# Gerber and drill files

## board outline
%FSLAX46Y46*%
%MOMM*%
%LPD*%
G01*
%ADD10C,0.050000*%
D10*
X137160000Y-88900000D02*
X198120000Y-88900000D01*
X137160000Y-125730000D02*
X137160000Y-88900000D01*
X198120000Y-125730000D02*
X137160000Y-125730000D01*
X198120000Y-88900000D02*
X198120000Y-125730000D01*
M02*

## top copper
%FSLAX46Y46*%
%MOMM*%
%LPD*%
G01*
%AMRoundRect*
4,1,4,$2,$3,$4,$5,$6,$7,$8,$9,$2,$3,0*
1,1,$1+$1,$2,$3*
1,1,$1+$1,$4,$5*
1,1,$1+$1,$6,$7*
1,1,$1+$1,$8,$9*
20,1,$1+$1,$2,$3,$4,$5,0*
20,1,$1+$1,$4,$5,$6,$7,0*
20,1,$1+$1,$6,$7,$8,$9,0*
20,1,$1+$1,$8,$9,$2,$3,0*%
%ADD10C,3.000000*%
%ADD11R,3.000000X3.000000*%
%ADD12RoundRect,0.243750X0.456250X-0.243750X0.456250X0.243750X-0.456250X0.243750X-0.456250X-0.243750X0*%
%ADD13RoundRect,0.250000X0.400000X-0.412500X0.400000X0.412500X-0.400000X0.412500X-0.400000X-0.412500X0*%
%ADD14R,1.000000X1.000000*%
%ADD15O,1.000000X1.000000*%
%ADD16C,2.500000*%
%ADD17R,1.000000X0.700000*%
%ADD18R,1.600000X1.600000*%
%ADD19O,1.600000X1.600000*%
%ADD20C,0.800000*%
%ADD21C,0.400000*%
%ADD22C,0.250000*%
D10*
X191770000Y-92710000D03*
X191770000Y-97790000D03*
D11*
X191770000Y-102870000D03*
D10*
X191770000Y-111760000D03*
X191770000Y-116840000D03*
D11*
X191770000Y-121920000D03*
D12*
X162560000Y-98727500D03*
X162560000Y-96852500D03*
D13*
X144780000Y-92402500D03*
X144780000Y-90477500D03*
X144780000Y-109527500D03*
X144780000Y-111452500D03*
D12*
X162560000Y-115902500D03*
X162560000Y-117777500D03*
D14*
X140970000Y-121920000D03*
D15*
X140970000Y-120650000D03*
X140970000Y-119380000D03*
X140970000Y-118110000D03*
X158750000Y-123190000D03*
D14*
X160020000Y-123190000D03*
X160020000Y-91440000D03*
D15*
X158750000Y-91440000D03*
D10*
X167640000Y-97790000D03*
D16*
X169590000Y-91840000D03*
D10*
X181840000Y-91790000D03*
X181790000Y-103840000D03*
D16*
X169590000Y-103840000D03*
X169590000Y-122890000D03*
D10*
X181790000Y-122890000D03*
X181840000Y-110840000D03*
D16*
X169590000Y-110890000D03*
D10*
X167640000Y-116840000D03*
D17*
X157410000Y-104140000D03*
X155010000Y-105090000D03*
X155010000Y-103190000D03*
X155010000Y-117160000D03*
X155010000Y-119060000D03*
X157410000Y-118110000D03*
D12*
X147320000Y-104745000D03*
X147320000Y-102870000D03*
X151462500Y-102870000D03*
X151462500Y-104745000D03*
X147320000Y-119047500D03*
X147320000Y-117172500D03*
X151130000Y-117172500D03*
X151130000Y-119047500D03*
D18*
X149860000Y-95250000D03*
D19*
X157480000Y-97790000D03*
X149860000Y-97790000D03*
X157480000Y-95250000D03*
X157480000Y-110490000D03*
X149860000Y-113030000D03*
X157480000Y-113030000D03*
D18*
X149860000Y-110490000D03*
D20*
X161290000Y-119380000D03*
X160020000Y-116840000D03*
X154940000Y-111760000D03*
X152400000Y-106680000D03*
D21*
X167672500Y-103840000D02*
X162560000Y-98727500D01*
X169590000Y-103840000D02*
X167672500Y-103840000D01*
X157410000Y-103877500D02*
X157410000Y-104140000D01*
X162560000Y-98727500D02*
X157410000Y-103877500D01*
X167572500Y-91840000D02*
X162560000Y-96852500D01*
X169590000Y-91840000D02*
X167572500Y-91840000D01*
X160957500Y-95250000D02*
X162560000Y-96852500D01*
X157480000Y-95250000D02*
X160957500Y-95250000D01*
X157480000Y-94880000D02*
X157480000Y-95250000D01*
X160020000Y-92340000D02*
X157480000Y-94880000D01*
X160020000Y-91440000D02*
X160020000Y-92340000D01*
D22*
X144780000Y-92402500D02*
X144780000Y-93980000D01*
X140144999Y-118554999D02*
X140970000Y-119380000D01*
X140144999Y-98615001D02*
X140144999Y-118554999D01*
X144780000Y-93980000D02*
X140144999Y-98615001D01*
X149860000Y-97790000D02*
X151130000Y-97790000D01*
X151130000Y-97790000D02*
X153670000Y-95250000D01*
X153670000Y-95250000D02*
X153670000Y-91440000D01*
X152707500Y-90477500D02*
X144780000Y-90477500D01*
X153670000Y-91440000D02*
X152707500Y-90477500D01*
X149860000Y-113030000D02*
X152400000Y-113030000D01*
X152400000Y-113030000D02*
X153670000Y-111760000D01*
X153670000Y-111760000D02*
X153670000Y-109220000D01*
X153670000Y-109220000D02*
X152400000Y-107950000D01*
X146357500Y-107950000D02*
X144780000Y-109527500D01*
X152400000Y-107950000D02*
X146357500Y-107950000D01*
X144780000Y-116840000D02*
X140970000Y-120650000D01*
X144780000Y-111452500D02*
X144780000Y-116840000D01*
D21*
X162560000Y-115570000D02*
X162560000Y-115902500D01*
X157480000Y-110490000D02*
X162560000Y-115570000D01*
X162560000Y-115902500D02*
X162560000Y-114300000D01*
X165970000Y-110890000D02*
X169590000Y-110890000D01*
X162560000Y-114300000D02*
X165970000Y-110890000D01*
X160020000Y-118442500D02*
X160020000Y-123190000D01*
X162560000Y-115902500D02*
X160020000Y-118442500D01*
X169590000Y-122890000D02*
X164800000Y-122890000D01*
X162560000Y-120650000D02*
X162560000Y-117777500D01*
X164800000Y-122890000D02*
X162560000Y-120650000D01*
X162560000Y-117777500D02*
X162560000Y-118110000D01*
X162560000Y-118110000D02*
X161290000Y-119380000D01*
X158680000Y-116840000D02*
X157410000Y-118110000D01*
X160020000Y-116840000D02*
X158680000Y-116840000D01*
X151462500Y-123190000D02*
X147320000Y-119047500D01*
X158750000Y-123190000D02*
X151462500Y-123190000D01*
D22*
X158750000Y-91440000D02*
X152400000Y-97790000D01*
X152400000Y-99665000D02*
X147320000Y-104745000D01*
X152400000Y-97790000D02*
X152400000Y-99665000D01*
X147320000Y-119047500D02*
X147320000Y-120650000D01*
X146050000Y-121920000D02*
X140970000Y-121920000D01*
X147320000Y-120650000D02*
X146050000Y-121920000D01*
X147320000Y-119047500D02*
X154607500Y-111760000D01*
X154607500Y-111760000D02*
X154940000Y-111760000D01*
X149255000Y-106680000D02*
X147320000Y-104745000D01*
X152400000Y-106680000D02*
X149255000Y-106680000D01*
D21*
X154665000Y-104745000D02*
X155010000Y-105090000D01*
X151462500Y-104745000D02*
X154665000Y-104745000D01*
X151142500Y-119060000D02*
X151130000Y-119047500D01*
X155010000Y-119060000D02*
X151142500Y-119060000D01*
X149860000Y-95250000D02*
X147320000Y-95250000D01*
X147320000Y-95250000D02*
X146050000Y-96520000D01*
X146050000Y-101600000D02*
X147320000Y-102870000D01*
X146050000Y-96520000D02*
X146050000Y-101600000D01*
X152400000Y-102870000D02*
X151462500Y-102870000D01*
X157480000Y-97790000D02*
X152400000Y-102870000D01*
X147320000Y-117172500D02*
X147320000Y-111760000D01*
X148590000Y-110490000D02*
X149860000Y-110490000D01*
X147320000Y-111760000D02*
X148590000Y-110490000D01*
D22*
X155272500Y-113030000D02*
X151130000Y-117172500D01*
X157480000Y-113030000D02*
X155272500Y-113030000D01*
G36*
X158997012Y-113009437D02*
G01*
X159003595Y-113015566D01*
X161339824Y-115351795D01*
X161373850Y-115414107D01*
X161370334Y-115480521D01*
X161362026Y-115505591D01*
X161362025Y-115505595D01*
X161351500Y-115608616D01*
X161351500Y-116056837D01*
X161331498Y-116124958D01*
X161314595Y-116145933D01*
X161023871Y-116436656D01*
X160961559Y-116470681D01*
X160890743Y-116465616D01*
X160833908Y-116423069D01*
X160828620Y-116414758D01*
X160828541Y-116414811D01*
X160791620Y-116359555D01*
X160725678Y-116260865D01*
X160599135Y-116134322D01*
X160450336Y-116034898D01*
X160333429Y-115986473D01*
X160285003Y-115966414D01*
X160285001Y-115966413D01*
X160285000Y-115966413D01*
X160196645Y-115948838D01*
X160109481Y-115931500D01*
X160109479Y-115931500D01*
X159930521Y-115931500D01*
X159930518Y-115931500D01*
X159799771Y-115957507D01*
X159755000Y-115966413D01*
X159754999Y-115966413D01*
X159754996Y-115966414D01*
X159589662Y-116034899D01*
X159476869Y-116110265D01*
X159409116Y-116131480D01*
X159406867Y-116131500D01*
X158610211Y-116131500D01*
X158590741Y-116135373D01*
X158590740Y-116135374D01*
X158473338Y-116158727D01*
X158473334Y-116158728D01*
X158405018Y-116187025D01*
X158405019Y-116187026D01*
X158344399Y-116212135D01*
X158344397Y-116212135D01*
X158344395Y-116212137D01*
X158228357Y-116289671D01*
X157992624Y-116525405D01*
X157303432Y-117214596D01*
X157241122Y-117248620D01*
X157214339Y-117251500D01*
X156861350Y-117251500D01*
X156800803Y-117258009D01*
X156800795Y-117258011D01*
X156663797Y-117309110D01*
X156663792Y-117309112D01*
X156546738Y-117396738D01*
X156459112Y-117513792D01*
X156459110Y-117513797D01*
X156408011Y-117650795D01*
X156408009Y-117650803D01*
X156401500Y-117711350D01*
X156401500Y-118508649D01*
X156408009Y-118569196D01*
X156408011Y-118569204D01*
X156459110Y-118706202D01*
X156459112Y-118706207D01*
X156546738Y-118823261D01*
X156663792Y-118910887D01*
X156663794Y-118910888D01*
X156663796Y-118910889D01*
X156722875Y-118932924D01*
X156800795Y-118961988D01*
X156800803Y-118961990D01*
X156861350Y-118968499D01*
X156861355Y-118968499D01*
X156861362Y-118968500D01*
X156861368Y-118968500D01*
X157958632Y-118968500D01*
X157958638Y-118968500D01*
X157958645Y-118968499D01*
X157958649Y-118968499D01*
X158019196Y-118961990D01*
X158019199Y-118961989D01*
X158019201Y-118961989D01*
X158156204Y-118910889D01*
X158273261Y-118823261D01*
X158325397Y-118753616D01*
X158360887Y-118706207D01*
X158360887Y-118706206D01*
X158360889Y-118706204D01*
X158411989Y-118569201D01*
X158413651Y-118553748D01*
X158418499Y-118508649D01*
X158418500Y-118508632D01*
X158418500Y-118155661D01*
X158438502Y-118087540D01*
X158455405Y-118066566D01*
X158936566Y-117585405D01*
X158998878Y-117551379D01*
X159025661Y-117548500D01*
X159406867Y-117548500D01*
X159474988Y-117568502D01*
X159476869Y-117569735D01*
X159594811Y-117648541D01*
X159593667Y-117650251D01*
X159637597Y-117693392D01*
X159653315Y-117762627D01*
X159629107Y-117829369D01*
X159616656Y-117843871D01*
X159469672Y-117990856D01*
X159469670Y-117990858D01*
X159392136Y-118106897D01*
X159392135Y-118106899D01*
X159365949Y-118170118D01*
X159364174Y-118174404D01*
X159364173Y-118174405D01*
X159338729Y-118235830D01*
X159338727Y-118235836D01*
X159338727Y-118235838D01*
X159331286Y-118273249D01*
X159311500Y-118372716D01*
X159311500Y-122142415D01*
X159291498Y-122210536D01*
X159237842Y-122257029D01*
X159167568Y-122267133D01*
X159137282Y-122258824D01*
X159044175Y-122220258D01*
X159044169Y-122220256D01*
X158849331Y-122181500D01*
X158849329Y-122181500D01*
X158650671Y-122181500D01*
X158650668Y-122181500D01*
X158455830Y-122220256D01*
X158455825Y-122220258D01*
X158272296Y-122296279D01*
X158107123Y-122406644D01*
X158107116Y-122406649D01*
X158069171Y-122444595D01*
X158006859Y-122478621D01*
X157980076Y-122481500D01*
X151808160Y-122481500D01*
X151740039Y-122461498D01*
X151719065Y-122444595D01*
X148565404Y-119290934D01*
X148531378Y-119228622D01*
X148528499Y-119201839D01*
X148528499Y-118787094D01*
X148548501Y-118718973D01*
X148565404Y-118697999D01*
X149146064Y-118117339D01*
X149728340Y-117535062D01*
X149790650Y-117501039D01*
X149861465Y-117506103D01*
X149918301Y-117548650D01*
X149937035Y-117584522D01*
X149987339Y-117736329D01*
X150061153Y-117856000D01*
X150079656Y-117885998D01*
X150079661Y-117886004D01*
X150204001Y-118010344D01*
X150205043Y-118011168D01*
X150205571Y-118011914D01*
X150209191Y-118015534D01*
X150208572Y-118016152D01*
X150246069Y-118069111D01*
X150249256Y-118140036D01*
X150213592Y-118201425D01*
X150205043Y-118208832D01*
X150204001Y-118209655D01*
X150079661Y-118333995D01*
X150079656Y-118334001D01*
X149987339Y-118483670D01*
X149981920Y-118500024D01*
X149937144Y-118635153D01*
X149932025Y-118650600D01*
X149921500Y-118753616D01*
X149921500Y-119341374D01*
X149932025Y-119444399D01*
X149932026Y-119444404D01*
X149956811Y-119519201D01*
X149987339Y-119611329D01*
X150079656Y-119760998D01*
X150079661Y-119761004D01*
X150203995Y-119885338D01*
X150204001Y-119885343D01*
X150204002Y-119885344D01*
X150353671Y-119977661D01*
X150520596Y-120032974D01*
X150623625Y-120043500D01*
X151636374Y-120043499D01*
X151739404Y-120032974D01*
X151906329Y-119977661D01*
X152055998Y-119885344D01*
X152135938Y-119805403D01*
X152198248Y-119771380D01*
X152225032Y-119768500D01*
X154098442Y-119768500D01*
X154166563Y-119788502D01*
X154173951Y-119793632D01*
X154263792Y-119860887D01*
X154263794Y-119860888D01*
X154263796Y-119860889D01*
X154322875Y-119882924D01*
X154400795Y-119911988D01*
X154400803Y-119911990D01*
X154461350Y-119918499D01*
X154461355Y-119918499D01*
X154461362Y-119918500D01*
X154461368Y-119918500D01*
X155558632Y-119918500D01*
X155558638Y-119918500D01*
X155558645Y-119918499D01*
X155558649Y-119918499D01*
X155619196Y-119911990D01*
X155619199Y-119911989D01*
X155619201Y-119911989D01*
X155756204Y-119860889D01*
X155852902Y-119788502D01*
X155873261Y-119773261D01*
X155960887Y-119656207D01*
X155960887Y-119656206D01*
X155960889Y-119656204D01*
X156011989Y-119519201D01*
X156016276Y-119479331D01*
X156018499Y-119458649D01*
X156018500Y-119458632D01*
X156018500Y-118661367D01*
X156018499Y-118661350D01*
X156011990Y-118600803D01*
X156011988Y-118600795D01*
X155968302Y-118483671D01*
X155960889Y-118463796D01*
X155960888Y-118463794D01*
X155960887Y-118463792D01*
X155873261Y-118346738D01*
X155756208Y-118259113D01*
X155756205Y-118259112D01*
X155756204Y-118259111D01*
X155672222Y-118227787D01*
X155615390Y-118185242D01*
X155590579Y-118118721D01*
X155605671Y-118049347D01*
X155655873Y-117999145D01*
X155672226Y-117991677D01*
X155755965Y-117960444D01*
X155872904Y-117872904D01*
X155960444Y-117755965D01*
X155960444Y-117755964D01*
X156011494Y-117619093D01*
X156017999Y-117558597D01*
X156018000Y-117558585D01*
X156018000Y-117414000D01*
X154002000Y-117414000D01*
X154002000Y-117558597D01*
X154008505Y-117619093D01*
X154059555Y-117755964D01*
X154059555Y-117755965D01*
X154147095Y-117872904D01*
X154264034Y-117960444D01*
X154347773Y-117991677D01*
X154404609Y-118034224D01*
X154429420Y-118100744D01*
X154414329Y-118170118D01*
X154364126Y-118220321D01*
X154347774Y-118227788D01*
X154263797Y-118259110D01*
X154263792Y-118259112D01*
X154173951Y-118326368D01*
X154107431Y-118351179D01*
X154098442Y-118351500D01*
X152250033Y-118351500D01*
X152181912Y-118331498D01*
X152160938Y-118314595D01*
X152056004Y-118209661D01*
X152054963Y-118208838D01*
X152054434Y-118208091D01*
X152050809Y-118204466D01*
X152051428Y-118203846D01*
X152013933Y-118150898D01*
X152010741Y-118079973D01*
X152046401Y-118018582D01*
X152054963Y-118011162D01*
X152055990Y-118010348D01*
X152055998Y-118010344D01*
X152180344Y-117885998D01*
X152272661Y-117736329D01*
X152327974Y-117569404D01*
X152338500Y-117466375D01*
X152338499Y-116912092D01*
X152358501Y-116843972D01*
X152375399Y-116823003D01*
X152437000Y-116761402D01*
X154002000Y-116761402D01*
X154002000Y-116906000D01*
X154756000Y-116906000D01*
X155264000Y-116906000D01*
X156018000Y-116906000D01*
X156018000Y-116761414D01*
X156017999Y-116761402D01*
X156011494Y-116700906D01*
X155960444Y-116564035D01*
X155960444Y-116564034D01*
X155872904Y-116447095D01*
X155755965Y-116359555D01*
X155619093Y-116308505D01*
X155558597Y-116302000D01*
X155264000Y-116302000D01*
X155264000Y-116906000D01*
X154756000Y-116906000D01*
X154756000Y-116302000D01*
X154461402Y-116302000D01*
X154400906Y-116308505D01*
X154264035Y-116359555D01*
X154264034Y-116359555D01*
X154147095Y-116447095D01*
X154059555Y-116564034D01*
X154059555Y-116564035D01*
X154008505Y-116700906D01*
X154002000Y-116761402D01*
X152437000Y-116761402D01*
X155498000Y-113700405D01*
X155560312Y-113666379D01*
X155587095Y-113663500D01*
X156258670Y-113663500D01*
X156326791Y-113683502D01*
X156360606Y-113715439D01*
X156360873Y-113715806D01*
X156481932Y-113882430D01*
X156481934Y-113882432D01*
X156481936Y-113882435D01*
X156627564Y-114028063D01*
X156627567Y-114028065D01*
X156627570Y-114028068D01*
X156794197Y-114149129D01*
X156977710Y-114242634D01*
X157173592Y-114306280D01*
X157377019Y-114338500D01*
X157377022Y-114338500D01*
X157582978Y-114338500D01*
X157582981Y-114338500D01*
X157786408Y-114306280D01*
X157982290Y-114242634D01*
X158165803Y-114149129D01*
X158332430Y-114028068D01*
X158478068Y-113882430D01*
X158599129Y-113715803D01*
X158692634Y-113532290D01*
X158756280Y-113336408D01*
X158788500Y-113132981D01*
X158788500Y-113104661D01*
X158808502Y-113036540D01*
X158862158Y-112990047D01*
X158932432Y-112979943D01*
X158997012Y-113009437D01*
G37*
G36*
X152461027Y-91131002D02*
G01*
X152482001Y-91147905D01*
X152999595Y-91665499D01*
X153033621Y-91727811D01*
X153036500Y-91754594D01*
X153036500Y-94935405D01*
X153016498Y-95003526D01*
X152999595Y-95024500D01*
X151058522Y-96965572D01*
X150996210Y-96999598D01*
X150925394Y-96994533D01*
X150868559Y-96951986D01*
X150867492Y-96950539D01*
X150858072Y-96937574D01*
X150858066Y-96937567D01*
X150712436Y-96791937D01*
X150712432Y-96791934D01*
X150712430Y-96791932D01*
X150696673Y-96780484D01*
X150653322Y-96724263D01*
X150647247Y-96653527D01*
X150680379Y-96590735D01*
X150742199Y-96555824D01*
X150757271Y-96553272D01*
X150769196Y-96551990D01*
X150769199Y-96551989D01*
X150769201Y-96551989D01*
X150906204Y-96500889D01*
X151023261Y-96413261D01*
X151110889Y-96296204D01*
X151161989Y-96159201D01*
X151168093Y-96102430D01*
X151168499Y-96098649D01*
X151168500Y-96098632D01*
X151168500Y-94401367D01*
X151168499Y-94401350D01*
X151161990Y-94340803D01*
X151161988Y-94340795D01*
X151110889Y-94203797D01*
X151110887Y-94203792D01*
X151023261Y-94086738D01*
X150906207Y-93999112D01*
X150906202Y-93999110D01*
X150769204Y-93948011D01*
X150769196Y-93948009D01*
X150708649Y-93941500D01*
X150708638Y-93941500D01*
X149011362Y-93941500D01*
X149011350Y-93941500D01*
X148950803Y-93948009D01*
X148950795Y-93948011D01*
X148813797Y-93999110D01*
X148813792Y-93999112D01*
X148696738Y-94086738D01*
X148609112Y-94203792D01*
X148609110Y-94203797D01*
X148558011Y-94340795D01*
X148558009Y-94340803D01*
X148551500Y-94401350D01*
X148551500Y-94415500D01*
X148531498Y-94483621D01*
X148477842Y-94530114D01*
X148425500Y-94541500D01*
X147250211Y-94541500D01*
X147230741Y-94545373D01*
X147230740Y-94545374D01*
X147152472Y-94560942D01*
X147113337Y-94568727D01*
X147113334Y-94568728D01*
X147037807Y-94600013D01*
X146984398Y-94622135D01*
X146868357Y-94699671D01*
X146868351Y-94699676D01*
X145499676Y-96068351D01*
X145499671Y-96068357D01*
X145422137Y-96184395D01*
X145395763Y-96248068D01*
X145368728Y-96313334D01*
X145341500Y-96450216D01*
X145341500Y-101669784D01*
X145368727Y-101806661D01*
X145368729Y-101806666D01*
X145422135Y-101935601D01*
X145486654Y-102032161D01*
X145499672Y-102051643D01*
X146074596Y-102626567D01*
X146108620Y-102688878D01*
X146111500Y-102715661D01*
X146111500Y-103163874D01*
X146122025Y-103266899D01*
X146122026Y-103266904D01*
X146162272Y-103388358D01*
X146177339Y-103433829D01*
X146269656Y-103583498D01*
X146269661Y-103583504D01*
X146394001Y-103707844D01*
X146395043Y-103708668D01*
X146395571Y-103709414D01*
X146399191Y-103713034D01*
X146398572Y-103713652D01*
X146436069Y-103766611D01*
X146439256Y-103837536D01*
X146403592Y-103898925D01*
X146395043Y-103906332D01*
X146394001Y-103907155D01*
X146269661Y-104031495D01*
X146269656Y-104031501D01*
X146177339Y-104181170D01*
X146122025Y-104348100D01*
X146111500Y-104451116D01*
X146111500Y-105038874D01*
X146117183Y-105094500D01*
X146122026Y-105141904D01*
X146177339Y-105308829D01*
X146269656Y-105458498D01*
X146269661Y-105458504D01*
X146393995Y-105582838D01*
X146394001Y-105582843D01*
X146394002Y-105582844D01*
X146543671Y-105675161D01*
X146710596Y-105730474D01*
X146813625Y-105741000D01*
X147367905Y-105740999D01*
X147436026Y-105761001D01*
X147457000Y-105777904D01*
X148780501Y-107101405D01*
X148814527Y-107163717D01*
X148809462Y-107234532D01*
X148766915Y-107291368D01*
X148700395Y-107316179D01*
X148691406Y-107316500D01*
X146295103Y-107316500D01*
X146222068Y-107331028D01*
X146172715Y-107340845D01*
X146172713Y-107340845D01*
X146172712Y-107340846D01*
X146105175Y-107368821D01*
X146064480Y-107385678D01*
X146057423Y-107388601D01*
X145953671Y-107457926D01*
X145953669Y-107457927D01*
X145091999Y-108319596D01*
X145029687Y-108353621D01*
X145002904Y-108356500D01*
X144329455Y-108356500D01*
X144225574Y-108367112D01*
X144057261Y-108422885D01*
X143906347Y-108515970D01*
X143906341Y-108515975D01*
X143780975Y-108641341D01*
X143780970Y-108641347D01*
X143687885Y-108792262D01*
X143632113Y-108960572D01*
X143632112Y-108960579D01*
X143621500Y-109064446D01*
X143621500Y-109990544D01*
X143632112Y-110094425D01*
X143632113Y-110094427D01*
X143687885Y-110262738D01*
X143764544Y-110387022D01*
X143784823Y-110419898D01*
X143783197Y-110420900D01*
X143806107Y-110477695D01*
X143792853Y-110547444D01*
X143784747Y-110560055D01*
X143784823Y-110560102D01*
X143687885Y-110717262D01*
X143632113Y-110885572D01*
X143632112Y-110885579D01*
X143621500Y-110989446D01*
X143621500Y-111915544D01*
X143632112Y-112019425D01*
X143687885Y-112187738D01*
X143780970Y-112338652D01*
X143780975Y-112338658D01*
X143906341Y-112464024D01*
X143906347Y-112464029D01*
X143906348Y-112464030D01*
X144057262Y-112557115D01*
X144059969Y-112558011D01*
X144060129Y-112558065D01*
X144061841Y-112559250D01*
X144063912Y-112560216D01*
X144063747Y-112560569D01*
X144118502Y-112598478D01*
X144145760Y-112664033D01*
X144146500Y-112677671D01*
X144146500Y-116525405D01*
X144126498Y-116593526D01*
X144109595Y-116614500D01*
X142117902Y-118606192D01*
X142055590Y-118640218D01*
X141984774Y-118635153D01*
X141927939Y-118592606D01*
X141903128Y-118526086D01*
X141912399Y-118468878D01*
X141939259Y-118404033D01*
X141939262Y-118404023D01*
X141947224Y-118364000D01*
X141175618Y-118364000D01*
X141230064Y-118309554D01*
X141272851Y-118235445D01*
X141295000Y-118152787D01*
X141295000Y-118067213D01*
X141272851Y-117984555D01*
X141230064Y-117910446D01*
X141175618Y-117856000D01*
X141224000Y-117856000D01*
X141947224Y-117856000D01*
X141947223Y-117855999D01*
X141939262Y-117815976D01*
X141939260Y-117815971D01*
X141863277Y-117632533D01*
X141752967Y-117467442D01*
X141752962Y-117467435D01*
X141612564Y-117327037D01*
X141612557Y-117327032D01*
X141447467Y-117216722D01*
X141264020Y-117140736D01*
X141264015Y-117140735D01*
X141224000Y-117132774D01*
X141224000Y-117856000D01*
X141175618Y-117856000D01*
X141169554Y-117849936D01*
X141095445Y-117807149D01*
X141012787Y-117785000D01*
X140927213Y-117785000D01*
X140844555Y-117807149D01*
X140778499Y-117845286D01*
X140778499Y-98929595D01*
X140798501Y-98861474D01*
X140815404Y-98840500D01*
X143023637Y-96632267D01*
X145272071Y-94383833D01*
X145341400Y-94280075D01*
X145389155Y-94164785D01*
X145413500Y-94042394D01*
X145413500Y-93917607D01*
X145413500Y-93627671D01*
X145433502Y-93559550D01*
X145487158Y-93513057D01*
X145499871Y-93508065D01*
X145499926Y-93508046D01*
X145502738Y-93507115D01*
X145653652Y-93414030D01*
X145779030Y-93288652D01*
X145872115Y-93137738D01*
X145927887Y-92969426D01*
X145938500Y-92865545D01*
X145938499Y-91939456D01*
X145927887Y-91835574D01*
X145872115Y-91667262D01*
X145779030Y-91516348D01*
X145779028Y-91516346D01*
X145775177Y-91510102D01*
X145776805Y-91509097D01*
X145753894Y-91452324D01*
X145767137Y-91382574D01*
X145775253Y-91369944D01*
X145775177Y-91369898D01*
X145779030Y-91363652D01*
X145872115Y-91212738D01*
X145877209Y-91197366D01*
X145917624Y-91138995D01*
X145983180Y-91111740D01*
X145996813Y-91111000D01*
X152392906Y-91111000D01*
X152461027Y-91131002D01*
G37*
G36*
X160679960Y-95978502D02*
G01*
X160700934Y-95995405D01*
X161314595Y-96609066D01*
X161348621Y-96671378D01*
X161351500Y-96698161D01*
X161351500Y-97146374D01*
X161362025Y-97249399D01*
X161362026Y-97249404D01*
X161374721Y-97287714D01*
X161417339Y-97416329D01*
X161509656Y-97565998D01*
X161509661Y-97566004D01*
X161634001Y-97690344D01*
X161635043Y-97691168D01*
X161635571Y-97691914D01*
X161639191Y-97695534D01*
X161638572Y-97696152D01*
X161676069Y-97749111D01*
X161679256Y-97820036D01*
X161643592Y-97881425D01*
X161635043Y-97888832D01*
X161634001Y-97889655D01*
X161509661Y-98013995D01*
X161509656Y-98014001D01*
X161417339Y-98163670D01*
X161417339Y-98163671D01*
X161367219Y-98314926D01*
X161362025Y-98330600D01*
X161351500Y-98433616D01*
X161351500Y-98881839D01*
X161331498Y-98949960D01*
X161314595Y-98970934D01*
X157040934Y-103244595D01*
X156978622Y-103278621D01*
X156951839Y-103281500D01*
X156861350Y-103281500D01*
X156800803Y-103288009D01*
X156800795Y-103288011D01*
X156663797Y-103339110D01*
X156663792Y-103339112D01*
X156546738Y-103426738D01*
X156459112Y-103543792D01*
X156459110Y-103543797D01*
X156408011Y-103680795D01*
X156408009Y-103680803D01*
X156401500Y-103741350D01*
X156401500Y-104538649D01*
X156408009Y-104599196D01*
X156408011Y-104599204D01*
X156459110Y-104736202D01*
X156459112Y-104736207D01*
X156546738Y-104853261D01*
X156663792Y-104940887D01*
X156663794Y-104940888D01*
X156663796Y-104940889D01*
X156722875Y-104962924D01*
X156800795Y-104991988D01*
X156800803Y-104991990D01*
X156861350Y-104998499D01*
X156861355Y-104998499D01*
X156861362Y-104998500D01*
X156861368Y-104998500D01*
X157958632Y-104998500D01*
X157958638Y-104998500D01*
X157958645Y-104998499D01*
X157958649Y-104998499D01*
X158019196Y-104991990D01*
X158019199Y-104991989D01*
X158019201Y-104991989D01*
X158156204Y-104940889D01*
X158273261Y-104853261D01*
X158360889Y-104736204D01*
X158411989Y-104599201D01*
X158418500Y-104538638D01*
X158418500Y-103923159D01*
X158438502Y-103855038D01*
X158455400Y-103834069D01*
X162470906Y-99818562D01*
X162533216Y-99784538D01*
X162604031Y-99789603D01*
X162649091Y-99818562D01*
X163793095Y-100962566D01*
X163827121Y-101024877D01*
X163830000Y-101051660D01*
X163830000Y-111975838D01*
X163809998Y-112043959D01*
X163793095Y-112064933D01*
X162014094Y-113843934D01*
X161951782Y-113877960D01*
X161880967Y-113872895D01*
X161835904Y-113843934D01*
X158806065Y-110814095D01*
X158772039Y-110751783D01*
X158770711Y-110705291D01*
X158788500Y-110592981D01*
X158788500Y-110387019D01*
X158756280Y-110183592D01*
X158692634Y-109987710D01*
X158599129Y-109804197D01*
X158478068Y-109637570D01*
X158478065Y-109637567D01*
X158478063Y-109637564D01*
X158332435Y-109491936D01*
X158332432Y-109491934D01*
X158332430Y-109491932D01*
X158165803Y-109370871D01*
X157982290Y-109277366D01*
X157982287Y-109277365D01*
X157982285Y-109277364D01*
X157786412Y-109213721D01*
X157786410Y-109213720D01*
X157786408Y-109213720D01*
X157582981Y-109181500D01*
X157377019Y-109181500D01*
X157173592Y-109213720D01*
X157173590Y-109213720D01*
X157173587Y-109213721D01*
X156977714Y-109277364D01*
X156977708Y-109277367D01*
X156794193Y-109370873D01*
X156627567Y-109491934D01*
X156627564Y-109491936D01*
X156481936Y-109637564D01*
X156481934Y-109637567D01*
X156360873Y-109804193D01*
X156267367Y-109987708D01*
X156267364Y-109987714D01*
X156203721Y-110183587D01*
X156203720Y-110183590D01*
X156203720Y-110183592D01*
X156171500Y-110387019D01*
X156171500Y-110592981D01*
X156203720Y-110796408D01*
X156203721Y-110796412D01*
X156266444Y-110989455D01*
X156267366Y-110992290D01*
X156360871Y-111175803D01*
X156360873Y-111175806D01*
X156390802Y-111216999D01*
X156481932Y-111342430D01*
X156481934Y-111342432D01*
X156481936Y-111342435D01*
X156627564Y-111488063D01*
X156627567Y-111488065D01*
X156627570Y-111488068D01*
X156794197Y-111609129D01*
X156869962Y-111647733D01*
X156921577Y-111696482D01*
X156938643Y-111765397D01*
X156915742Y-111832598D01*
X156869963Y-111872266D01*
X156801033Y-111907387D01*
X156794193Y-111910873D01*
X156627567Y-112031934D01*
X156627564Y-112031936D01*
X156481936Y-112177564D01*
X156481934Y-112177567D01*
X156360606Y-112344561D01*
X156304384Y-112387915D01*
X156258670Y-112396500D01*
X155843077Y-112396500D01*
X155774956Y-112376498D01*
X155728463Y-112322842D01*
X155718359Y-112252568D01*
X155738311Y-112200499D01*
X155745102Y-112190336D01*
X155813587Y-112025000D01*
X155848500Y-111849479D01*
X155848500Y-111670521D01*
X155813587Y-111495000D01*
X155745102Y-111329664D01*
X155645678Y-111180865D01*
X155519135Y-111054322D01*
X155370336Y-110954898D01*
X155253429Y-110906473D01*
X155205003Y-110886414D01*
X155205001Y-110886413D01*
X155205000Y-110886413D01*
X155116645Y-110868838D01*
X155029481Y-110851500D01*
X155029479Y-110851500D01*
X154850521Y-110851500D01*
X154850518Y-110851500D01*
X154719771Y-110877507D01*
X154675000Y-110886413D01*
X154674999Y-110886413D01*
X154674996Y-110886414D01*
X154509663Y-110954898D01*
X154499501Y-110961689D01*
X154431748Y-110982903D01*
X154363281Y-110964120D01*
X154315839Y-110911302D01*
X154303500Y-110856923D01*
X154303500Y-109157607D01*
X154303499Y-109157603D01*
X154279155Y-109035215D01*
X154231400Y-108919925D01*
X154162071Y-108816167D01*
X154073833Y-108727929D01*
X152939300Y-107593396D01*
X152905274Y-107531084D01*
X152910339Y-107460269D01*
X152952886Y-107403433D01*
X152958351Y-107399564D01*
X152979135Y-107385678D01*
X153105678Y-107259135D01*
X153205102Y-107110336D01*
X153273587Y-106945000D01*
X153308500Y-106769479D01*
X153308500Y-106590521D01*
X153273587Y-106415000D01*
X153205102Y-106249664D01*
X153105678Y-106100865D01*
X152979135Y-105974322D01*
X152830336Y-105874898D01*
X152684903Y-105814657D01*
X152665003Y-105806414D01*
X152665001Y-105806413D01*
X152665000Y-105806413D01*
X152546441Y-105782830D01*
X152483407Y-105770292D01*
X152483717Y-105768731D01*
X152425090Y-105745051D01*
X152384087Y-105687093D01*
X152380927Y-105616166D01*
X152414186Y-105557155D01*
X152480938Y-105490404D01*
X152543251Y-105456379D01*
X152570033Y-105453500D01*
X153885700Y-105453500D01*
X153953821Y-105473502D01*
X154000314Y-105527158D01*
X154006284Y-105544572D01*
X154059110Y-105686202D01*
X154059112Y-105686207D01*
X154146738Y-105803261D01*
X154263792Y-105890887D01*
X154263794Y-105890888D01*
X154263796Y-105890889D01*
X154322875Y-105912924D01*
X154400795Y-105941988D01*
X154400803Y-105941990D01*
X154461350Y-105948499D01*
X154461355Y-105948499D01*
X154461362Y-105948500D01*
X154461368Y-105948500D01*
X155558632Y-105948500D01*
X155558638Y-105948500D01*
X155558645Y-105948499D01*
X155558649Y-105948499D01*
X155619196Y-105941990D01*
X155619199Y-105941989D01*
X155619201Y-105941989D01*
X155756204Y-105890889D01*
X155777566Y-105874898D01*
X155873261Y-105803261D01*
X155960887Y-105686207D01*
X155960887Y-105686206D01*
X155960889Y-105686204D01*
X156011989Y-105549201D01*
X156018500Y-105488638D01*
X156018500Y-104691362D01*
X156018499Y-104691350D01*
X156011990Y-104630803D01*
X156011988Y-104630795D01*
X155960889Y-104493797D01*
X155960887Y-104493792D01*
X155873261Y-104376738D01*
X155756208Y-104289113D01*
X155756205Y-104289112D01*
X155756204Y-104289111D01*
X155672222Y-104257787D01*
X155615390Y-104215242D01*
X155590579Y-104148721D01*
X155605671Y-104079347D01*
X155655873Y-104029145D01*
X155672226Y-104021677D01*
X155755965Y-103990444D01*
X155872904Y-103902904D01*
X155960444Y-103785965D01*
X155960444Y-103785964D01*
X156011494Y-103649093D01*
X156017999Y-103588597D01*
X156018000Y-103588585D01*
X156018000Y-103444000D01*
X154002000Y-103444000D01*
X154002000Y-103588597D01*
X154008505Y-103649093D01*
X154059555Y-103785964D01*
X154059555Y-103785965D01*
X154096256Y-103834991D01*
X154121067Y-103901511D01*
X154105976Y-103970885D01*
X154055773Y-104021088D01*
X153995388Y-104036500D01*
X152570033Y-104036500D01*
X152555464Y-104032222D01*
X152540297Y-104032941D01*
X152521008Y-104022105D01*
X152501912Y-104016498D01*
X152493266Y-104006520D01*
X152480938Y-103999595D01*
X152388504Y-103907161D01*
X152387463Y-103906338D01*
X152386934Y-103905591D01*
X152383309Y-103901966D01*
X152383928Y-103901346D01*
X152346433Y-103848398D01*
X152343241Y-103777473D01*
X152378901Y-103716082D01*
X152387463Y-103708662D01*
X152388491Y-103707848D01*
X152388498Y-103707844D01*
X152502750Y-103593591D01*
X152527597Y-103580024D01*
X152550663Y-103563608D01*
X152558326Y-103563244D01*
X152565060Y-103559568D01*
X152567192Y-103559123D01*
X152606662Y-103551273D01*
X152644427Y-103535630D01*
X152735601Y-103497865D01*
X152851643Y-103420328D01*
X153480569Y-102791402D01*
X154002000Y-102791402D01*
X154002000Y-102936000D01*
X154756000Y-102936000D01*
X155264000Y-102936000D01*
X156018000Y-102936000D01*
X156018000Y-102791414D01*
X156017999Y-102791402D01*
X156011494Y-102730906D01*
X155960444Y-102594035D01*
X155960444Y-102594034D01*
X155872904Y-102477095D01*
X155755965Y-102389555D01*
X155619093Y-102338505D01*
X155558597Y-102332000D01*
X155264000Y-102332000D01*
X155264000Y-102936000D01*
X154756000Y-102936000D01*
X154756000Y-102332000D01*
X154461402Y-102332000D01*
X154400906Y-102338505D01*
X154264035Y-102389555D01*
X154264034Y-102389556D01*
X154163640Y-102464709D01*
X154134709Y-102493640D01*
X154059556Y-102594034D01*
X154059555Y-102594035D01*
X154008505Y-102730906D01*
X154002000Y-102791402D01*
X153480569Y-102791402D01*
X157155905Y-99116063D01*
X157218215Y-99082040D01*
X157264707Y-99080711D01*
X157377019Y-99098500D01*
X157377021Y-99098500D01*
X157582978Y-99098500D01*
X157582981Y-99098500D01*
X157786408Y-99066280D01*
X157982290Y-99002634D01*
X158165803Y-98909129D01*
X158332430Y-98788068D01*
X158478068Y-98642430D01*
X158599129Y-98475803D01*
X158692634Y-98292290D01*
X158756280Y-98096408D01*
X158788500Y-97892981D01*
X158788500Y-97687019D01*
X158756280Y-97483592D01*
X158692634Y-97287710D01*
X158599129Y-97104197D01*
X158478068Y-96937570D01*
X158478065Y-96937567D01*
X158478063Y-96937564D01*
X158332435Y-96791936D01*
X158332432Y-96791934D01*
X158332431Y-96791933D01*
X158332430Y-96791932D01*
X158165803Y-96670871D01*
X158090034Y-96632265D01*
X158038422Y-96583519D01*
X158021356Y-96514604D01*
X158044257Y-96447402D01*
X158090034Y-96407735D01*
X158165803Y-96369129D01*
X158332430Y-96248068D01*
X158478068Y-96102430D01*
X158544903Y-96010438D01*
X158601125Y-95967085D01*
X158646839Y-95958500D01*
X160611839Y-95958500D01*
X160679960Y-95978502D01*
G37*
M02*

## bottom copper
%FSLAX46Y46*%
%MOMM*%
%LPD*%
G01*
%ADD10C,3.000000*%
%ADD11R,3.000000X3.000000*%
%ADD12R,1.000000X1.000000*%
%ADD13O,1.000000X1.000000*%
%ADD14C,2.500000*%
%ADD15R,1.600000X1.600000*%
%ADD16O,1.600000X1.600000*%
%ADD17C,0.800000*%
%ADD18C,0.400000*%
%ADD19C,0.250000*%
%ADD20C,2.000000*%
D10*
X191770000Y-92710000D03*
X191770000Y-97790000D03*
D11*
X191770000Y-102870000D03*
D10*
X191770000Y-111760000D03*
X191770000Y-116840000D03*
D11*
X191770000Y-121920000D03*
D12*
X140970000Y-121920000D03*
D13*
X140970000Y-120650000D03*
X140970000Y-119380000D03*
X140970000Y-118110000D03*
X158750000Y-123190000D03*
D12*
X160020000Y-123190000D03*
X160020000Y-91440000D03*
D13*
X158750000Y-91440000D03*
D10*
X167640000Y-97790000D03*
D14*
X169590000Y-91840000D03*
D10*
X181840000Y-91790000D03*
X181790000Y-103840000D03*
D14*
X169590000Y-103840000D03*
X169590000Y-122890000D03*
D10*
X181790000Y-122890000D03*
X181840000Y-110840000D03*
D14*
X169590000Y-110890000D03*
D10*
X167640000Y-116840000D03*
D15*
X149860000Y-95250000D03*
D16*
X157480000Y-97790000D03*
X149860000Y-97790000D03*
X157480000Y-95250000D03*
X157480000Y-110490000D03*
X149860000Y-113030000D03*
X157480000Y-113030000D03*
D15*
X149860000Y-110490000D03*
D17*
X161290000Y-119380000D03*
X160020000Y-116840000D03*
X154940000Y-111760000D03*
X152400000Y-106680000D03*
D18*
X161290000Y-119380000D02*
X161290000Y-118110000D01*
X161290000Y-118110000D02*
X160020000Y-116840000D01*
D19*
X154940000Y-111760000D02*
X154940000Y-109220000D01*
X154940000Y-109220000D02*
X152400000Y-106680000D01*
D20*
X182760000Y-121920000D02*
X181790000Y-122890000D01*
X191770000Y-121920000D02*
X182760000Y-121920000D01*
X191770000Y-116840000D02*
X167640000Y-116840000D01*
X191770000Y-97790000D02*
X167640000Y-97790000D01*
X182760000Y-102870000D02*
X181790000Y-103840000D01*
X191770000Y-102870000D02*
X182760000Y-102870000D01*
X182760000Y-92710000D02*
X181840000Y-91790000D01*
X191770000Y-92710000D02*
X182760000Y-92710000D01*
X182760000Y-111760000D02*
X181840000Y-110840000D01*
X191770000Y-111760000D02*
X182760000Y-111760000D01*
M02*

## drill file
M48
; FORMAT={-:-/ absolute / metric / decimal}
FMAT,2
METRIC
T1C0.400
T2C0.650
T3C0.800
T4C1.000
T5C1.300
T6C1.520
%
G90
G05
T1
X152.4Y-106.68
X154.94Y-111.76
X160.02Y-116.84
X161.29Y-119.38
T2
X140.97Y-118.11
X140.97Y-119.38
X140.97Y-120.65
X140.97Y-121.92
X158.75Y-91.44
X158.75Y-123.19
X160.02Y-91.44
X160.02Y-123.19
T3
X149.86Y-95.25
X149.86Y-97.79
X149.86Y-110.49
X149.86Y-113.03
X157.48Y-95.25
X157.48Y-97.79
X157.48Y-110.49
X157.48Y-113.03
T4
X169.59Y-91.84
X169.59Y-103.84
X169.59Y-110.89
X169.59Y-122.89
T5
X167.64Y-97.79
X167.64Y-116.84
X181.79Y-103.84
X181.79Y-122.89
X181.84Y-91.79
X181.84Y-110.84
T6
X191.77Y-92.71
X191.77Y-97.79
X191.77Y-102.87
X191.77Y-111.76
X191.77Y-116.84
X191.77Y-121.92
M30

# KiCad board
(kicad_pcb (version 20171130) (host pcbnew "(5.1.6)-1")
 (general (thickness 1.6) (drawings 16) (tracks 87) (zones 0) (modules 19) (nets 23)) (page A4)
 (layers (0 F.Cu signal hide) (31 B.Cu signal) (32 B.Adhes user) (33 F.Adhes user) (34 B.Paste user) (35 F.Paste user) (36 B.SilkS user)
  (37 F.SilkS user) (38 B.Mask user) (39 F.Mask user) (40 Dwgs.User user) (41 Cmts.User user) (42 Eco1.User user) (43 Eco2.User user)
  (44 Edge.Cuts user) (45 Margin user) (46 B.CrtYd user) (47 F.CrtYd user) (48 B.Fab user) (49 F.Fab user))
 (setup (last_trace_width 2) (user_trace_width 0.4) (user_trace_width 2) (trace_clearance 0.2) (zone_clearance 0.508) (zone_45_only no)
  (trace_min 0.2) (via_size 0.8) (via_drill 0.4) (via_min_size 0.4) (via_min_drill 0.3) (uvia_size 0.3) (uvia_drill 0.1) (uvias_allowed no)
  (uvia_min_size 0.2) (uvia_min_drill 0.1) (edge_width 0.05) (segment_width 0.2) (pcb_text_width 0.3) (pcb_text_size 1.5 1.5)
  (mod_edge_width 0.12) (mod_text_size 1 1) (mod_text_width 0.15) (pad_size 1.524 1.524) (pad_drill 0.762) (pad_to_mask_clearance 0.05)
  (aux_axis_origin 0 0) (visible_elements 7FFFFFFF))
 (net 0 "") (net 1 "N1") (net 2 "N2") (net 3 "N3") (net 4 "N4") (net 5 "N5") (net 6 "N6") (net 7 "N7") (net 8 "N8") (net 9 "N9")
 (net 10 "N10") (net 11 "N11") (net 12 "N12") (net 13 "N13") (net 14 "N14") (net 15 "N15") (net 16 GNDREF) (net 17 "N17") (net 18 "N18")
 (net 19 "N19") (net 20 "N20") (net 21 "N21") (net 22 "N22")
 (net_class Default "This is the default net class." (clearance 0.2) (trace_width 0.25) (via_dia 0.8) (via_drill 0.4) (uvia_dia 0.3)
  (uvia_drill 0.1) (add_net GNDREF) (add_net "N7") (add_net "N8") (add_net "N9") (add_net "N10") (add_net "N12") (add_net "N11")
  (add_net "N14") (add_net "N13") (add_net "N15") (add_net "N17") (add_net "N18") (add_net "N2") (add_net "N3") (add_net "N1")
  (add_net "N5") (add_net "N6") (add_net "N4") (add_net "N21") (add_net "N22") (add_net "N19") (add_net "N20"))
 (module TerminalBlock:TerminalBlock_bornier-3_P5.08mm (layer F.Cu) (at 191.77 102.87 90)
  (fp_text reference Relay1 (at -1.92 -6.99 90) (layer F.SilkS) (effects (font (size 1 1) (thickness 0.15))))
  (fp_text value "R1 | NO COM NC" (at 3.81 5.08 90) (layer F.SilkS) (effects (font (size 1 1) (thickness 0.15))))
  (pad 3 thru_hole circle (at 10.16 0 90) (size 3 3) (drill 1.52) (layers *.Cu *.Mask) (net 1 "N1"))
  (pad 2 thru_hole circle (at 5.08 0 90) (size 3 3) (drill 1.52) (layers *.Cu *.Mask) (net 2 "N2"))
  (pad 1 thru_hole rect (at 0 0 90) (size 3 3) (drill 1.52) (layers *.Cu *.Mask) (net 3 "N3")))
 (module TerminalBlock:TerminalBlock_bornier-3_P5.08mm (layer F.Cu) (at 191.77 121.92 90)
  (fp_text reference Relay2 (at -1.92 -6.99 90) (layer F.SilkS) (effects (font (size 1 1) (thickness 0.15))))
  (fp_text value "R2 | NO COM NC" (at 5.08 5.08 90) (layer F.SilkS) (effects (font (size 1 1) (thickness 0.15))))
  (pad 3 thru_hole circle (at 10.16 0 90) (size 3 3) (drill 1.52) (layers *.Cu *.Mask) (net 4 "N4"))
  (pad 2 thru_hole circle (at 5.08 0 90) (size 3 3) (drill 1.52) (layers *.Cu *.Mask) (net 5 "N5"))
  (pad 1 thru_hole rect (at 0 0 90) (size 3 3) (drill 1.52) (layers *.Cu *.Mask) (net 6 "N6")))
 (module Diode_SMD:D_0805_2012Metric (layer F.Cu) (at 162.56 97.79 90)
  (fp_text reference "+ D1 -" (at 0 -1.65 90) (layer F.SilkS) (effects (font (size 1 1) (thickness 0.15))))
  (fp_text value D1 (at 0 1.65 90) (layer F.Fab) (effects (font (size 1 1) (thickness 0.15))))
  (pad 1 smd roundrect (at -0.9375 0 90) (size 0.975 1.4) (layers F.Cu F.Paste F.Mask) (roundrect_rratio 0.25) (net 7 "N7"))
  (pad 2 smd roundrect (at 0.9375 0 90) (size 0.975 1.4) (layers F.Cu F.Paste F.Mask) (roundrect_rratio 0.25) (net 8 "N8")))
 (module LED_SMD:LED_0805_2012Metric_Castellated (layer F.Cu) (at 144.78 91.44 90)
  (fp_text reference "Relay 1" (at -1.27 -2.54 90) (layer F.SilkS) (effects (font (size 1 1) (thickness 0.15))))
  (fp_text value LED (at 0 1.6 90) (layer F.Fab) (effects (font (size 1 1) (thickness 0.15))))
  (pad 1 smd roundrect (at -0.9625 0 90) (size 1.325 1.3) (layers F.Cu F.Paste F.Mask) (roundrect_rratio 0.192308) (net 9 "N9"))
  (pad 2 smd roundrect (at 0.9625 0 90) (size 1.325 1.3) (layers F.Cu F.Paste F.Mask) (roundrect_rratio 0.192308) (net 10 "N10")))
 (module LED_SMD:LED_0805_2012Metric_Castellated (layer F.Cu) (at 144.78 110.49 90)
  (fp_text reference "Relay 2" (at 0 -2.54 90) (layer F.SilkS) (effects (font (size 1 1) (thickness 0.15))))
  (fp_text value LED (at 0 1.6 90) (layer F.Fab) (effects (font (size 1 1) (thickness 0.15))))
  (pad 2 smd roundrect (at 0.9625 0 90) (size 1.325 1.3) (layers F.Cu F.Paste F.Mask) (roundrect_rratio 0.192308) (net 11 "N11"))
  (pad 1 smd roundrect (at -0.9625 0 90) (size 1.325 1.3) (layers F.Cu F.Paste F.Mask) (roundrect_rratio 0.192308) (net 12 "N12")))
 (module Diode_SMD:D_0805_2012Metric (layer F.Cu) (at 162.56 116.84 90)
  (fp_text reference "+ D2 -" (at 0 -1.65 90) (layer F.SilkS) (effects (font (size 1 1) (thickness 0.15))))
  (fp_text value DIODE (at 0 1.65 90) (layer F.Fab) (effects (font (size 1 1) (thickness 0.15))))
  (pad 2 smd roundrect (at 0.9375 0 90) (size 0.975 1.4) (layers F.Cu F.Paste F.Mask) (roundrect_rratio 0.25) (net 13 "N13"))
  (pad 1 smd roundrect (at -0.9375 0 90) (size 0.975 1.4) (layers F.Cu F.Paste F.Mask) (roundrect_rratio 0.25) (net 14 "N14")))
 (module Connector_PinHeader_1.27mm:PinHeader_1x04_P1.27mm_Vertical (layer F.Cu) (at 140.97 121.92 180)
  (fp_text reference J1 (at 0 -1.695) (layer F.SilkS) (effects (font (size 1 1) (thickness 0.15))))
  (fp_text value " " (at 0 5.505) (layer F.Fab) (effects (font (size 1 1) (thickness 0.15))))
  (pad 1 thru_hole rect (at 0 0 180) (size 1 1) (drill 0.65) (layers *.Cu *.Mask) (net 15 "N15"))
  (pad 2 thru_hole oval (at 0 1.27 180) (size 1 1) (drill 0.65) (layers *.Cu *.Mask) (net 12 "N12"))
  (pad 3 thru_hole oval (at 0 2.54 180) (size 1 1) (drill 0.65) (layers *.Cu *.Mask) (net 9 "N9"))
  (pad 4 thru_hole oval (at 0 3.81 180) (size 1 1) (drill 0.65) (layers *.Cu *.Mask) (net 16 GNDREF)))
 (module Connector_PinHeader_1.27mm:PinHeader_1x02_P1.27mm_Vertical (layer F.Cu) (at 160.02 123.19 270)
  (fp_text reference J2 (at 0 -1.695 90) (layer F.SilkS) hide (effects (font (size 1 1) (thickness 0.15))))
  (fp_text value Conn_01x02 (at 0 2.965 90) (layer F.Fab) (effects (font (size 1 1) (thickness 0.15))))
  (pad 2 thru_hole oval (at 0 1.27 270) (size 1 1) (drill 0.65) (layers *.Cu *.Mask) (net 15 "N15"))
  (pad 1 thru_hole rect (at 0 0 270) (size 1 1) (drill 0.65) (layers *.Cu *.Mask) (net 13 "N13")))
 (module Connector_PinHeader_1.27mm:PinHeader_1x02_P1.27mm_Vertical (layer F.Cu) (at 160.02 91.44 270)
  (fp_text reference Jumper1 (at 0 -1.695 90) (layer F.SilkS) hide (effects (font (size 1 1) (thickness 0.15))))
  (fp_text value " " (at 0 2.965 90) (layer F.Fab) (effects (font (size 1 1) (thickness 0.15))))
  (pad 1 thru_hole rect (at 0 0 270) (size 1 1) (drill 0.65) (layers *.Cu *.Mask) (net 8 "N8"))
  (pad 2 thru_hole oval (at 0 1.27 270) (size 1 1) (drill 0.65) (layers *.Cu *.Mask) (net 15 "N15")))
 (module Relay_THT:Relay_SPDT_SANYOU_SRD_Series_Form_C (layer F.Cu) (at 167.64 97.79)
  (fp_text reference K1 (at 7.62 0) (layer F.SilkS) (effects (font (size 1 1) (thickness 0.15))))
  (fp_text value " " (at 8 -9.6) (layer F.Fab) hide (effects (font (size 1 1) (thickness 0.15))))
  (pad 1 thru_hole circle (at 0 0 90) (size 3 3) (drill 1.3) (layers *.Cu *.Mask) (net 2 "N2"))
  (pad 5 thru_hole circle (at 1.95 -5.95 90) (size 2.5 2.5) (drill 1) (layers *.Cu *.Mask) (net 8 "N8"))
  (pad 4 thru_hole circle (at 14.2 -6 90) (size 3 3) (drill 1.3) (layers *.Cu *.Mask) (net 1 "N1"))
  (pad 3 thru_hole circle (at 14.15 6.05 90) (size 3 3) (drill 1.3) (layers *.Cu *.Mask) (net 3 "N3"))
  (pad 2 thru_hole circle (at 1.95 6.05 90) (size 2.5 2.5) (drill 1) (layers *.Cu *.Mask) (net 7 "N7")))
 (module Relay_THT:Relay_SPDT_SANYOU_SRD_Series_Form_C (layer F.Cu) (at 167.64 116.84)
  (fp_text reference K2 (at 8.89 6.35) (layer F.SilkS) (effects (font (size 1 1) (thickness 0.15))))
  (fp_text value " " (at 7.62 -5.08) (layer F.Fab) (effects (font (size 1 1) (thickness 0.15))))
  (pad 2 thru_hole circle (at 1.95 6.05 90) (size 2.5 2.5) (drill 1) (layers *.Cu *.Mask) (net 14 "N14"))
  (pad 3 thru_hole circle (at 14.15 6.05 90) (size 3 3) (drill 1.3) (layers *.Cu *.Mask) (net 6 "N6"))
  (pad 4 thru_hole circle (at 14.2 -6 90) (size 3 3) (drill 1.3) (layers *.Cu *.Mask) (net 4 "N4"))
  (pad 5 thru_hole circle (at 1.95 -5.95 90) (size 2.5 2.5) (drill 1) (layers *.Cu *.Mask) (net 13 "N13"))
  (pad 1 thru_hole circle (at 0 0 90) (size 3 3) (drill 1.3) (layers *.Cu *.Mask) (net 5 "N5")))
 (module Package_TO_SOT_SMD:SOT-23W (layer F.Cu) (at 156.21 104.14)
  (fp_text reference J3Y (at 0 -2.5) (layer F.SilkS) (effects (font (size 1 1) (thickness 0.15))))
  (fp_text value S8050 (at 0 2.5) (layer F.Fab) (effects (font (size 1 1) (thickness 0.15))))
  (pad 3 smd rect (at 1.2 0) (size 1 0.7) (layers F.Cu F.Paste F.Mask) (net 7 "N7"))
  (pad 2 smd rect (at -1.2 0.95) (size 1 0.7) (layers F.Cu F.Paste F.Mask) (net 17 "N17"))
  (pad 1 smd rect (at -1.2 -0.95) (size 1 0.7) (layers F.Cu F.Paste F.Mask) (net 16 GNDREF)))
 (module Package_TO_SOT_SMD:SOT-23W (layer F.Cu) (at 156.21 118.11)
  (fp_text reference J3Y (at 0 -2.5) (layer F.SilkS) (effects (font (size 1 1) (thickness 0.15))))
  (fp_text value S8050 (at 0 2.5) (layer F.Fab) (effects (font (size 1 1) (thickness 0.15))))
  (pad 1 smd rect (at -1.2 -0.95) (size 1 0.7) (layers F.Cu F.Paste F.Mask) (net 16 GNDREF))
  (pad 2 smd rect (at -1.2 0.95) (size 1 0.7) (layers F.Cu F.Paste F.Mask) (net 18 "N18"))
  (pad 3 smd rect (at 1.2 0) (size 1 0.7) (layers F.Cu F.Paste F.Mask) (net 14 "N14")))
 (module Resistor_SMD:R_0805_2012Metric (layer F.Cu) (at 147.32 103.8075 90)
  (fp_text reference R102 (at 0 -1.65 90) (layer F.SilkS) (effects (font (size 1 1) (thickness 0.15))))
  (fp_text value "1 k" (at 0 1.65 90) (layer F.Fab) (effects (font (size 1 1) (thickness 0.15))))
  (pad 1 smd roundrect (at -0.9375 0 90) (size 0.975 1.4) (layers F.Cu F.Paste F.Mask) (roundrect_rratio 0.25) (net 15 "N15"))
  (pad 2 smd roundrect (at 0.9375 0 90) (size 0.975 1.4) (layers F.Cu F.Paste F.Mask) (roundrect_rratio 0.25) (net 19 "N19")))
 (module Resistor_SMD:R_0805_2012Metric (layer F.Cu) (at 151.4625 103.8075 90)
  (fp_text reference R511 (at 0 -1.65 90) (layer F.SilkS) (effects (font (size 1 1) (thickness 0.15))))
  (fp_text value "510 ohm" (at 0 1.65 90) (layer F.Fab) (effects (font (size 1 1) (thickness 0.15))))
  (pad 2 smd roundrect (at 0.9375 0 90) (size 0.975 1.4) (layers F.Cu F.Paste F.Mask) (roundrect_rratio 0.25) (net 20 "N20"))
  (pad 1 smd roundrect (at -0.9375 0 90) (size 0.975 1.4) (layers F.Cu F.Paste F.Mask) (roundrect_rratio 0.25) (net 17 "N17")))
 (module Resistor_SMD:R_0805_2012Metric (layer F.Cu) (at 147.32 118.11 90)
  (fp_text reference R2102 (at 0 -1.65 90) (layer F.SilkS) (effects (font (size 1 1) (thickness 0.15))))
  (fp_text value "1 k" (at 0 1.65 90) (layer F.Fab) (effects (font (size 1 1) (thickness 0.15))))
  (pad 1 smd roundrect (at -0.9375 0 90) (size 0.975 1.4) (layers F.Cu F.Paste F.Mask) (roundrect_rratio 0.25) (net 15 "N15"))
  (pad 2 smd roundrect (at 0.9375 0 90) (size 0.975 1.4) (layers F.Cu F.Paste F.Mask) (roundrect_rratio 0.25) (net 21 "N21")))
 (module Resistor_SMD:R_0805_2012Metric (layer F.Cu) (at 151.13 118.11 90)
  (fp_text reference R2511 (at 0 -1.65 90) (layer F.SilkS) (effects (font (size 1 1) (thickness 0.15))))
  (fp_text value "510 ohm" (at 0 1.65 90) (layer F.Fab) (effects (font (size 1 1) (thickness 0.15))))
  (pad 2 smd roundrect (at 0.9375 0 90) (size 0.975 1.4) (layers F.Cu F.Paste F.Mask) (roundrect_rratio 0.25) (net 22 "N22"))
  (pad 1 smd roundrect (at -0.9375 0 90) (size 0.975 1.4) (layers F.Cu F.Paste F.Mask) (roundrect_rratio 0.25) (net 18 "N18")))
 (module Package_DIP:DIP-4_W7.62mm (layer F.Cu) (at 149.86 95.25)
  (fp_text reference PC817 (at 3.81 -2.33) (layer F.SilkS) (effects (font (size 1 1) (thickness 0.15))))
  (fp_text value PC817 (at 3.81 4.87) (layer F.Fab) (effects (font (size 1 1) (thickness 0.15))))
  (pad 1 thru_hole rect (at 0 0) (size 1.6 1.6) (drill 0.8) (layers *.Cu *.Mask) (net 19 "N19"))
  (pad 3 thru_hole oval (at 7.62 2.54) (size 1.6 1.6) (drill 0.8) (layers *.Cu *.Mask) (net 20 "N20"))
  (pad 2 thru_hole oval (at 0 2.54) (size 1.6 1.6) (drill 0.8) (layers *.Cu *.Mask) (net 10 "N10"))
  (pad 4 thru_hole oval (at 7.62 0) (size 1.6 1.6) (drill 0.8) (layers *.Cu *.Mask) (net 8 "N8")))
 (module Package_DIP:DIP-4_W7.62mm (layer F.Cu) (at 149.86 110.49)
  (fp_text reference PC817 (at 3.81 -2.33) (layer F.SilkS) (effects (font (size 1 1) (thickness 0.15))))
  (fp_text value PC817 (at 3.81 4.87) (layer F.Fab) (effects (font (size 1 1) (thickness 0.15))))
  (pad 4 thru_hole oval (at 7.62 0) (size 1.6 1.6) (drill 0.8) (layers *.Cu *.Mask) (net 13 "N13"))
  (pad 2 thru_hole oval (at 0 2.54) (size 1.6 1.6) (drill 0.8) (layers *.Cu *.Mask) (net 11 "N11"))
  (pad 3 thru_hole oval (at 7.62 2.54) (size 1.6 1.6) (drill 0.8) (layers *.Cu *.Mask) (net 22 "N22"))
  (pad 1 thru_hole rect (at 0 0) (size 1.6 1.6) (drill 0.8) (layers *.Cu *.Mask) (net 21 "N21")))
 (gr_line (start 137.16 88.9) (end 198.12 88.9) (layer Edge.Cuts) (width 0.05))
 (gr_line (start 137.16 125.73) (end 137.16 88.9) (layer Edge.Cuts) (width 0.05))
 (gr_line (start 198.12 125.73) (end 137.16 125.73) (layer Edge.Cuts) (width 0.05))
 (gr_line (start 198.12 88.9) (end 198.12 125.73) (layer Edge.Cuts) (width 0.05))
 (segment (start 167.6725 103.84) (end 162.56 98.7275) (width 0.4) (layer F.Cu) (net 7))
 (segment (start 169.59 103.84) (end 167.6725 103.84) (width 0.4) (layer F.Cu) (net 7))
 (segment (start 157.41 103.8775) (end 157.41 104.14) (width 0.4) (layer F.Cu) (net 7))
 (segment (start 162.56 98.7275) (end 157.41 103.8775) (width 0.4) (layer F.Cu) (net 7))
 (segment (start 167.5725 91.84) (end 162.56 96.8525) (width 0.4) (layer F.Cu) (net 8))
 (segment (start 169.59 91.84) (end 167.5725 91.84) (width 0.4) (layer F.Cu) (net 8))
 (segment (start 160.9575 95.25) (end 162.56 96.8525) (width 0.4) (layer F.Cu) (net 8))
 (segment (start 157.48 95.25) (end 160.9575 95.25) (width 0.4) (layer F.Cu) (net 8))
 (segment (start 157.48 94.88) (end 157.48 95.25) (width 0.4) (layer F.Cu) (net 8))
 (segment (start 160.02 92.34) (end 157.48 94.88) (width 0.4) (layer F.Cu) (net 8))
 (segment (start 160.02 91.44) (end 160.02 92.34) (width 0.4) (layer F.Cu) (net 8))
 (segment (start 144.78 92.4025) (end 144.78 93.98) (width 0.25) (layer F.Cu) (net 9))
 (segment (start 140.144999 118.554999) (end 140.97 119.38) (width 0.25) (layer F.Cu) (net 9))
 (segment (start 140.144999 98.615001) (end 140.144999 118.554999) (width 0.25) (layer F.Cu) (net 9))
 (segment (start 144.78 93.98) (end 140.144999 98.615001) (width 0.25) (layer F.Cu) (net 9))
 (segment (start 149.86 97.79) (end 151.13 97.79) (width 0.25) (layer F.Cu) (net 10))
 (segment (start 151.13 97.79) (end 153.67 95.25) (width 0.25) (layer F.Cu) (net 10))
 (segment (start 153.67 95.25) (end 153.67 91.44) (width 0.25) (layer F.Cu) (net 10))
 (segment (start 152.7075 90.4775) (end 144.78 90.4775) (width 0.25) (layer F.Cu) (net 10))
 (segment (start 153.67 91.44) (end 152.7075 90.4775) (width 0.25) (layer F.Cu) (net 10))
 (segment (start 149.86 113.03) (end 152.4 113.03) (width 0.25) (layer F.Cu) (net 11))
 (segment (start 152.4 113.03) (end 153.67 111.76) (width 0.25) (layer F.Cu) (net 11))
 (segment (start 153.67 111.76) (end 153.67 109.22) (width 0.25) (layer F.Cu) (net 11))
 (segment (start 153.67 109.22) (end 152.4 107.95) (width 0.25) (layer F.Cu) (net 11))
 (segment (start 146.3575 107.95) (end 144.78 109.5275) (width 0.25) (layer F.Cu) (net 11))
 (segment (start 152.4 107.95) (end 146.3575 107.95) (width 0.25) (layer F.Cu) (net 11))
 (segment (start 144.78 116.84) (end 140.97 120.65) (width 0.25) (layer F.Cu) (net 12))
 (segment (start 144.78 111.4525) (end 144.78 116.84) (width 0.25) (layer F.Cu) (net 12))
 (segment (start 162.56 115.57) (end 162.56 115.9025) (width 0.4) (layer F.Cu) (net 13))
 (segment (start 157.48 110.49) (end 162.56 115.57) (width 0.4) (layer F.Cu) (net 13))
 (segment (start 162.56 115.9025) (end 162.56 114.3) (width 0.4) (layer F.Cu) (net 13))
 (segment (start 165.97 110.89) (end 169.59 110.89) (width 0.4) (layer F.Cu) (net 13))
 (segment (start 162.56 114.3) (end 165.97 110.89) (width 0.4) (layer F.Cu) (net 13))
 (segment (start 160.02 118.4425) (end 160.02 123.19) (width 0.4) (layer F.Cu) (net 13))
 (segment (start 162.56 115.9025) (end 160.02 118.4425) (width 0.4) (layer F.Cu) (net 13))
 (segment (start 169.59 122.89) (end 164.8 122.89) (width 0.4) (layer F.Cu) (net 14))
 (segment (start 162.56 120.65) (end 162.56 117.7775) (width 0.4) (layer F.Cu) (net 14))
 (segment (start 164.8 122.89) (end 162.56 120.65) (width 0.4) (layer F.Cu) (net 14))
 (via (at 161.29 119.38) (size 0.8) (drill 0.4) (layers F.Cu B.Cu) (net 14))
 (segment (start 162.56 117.7775) (end 162.56 118.11) (width 0.4) (layer F.Cu) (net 14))
 (segment (start 162.56 118.11) (end 161.29 119.38) (width 0.4) (layer F.Cu) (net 14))
 (via (at 160.02 116.84) (size 0.8) (drill 0.4) (layers F.Cu B.Cu) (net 14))
 (segment (start 161.29 119.38) (end 161.29 118.11) (width 0.4) (layer B.Cu) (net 14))
 (segment (start 161.29 118.11) (end 160.02 116.84) (width 0.4) (layer B.Cu) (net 14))
 (segment (start 158.68 116.84) (end 157.41 118.11) (width 0.4) (layer F.Cu) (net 14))
 (segment (start 160.02 116.84) (end 158.68 116.84) (width 0.4) (layer F.Cu) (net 14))
 (segment (start 151.4625 123.19) (end 147.32 119.0475) (width 0.4) (layer F.Cu) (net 15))
 (segment (start 158.75 123.19) (end 151.4625 123.19) (width 0.4) (layer F.Cu) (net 15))
 (segment (start 158.75 91.44) (end 152.4 97.79) (width 0.25) (layer F.Cu) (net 15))
 (segment (start 152.4 99.665) (end 147.32 104.745) (width 0.25) (layer F.Cu) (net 15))
 (segment (start 152.4 97.79) (end 152.4 99.665) (width 0.25) (layer F.Cu) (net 15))
 (segment (start 147.32 119.0475) (end 147.32 120.65) (width 0.25) (layer F.Cu) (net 15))
 (segment (start 146.05 121.92) (end 140.97 121.92) (width 0.25) (layer F.Cu) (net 15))
 (segment (start 147.32 120.65) (end 146.05 121.92) (width 0.25) (layer F.Cu) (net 15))
 (segment (start 147.32 119.0475) (end 154.6075 111.76) (width 0.25) (layer F.Cu) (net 15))
 (via (at 154.94 111.76) (size 0.8) (drill 0.4) (layers F.Cu B.Cu) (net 15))
 (segment (start 154.6075 111.76) (end 154.94 111.76) (width 0.25) (layer F.Cu) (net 15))
 (segment (start 154.94 111.76) (end 154.94 109.22) (width 0.25) (layer B.Cu) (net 15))
 (via (at 152.4 106.68) (size 0.8) (drill 0.4) (layers F.Cu B.Cu) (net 15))
 (segment (start 154.94 109.22) (end 152.4 106.68) (width 0.25) (layer B.Cu) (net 15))
 (segment (start 149.255 106.68) (end 147.32 104.745) (width 0.25) (layer F.Cu) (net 15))
 (segment (start 152.4 106.68) (end 149.255 106.68) (width 0.25) (layer F.Cu) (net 15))
 (segment (start 182.76 121.92) (end 181.79 122.89) (width 2) (layer B.Cu) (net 6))
 (segment (start 191.77 121.92) (end 182.76 121.92) (width 2) (layer B.Cu) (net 6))
 (segment (start 191.77 116.84) (end 167.64 116.84) (width 2) (layer B.Cu) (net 5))
 (segment (start 191.77 97.79) (end 167.64 97.79) (width 2) (layer B.Cu) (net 2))
 (segment (start 182.76 102.87) (end 181.79 103.84) (width 2) (layer B.Cu) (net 3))
 (segment (start 191.77 102.87) (end 182.76 102.87) (width 2) (layer B.Cu) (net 3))
 (segment (start 154.665 104.745) (end 155.01 105.09) (width 0.4) (layer F.Cu) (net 17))
 (segment (start 151.4625 104.745) (end 154.665 104.745) (width 0.4) (layer F.Cu) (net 17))
 (segment (start 151.1425 119.06) (end 151.13 119.0475) (width 0.4) (layer F.Cu) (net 18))
 (segment (start 155.01 119.06) (end 151.1425 119.06) (width 0.4) (layer F.Cu) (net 18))
 (segment (start 149.86 95.25) (end 147.32 95.25) (width 0.4) (layer F.Cu) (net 19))
 (segment (start 147.32 95.25) (end 146.05 96.52) (width 0.4) (layer F.Cu) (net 19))
 (segment (start 146.05 101.6) (end 147.32 102.87) (width 0.4) (layer F.Cu) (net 19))
 (segment (start 146.05 96.52) (end 146.05 101.6) (width 0.4) (layer F.Cu) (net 19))
 (segment (start 152.4 102.87) (end 151.4625 102.87) (width 0.4) (layer F.Cu) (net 20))
 (segment (start 157.48 97.79) (end 152.4 102.87) (width 0.4) (layer F.Cu) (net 20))
 (segment (start 182.76 92.71) (end 181.84 91.79) (width 2) (layer B.Cu) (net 1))
 (segment (start 191.77 92.71) (end 182.76 92.71) (width 2) (layer B.Cu) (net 1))
 (segment (start 182.76 111.76) (end 181.84 110.84) (width 2) (layer B.Cu) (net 4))
 (segment (start 191.77 111.76) (end 182.76 111.76) (width 2) (layer B.Cu) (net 4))
 (segment (start 147.32 117.1725) (end 147.32 111.76) (width 0.4) (layer F.Cu) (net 21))
 (segment (start 148.59 110.49) (end 149.86 110.49) (width 0.4) (layer F.Cu) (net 21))
 (segment (start 147.32 111.76) (end 148.59 110.49) (width 0.4) (layer F.Cu) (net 21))
 (segment (start 155.2725 113.03) (end 151.13 117.1725) (width 0.25) (layer F.Cu) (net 22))
 (segment (start 157.48 113.03) (end 155.2725 113.03) (width 0.25) (layer F.Cu) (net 22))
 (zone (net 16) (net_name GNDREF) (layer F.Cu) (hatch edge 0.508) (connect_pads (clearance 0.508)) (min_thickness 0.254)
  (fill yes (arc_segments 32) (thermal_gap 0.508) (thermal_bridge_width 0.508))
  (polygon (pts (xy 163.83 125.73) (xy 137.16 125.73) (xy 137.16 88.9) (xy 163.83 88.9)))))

